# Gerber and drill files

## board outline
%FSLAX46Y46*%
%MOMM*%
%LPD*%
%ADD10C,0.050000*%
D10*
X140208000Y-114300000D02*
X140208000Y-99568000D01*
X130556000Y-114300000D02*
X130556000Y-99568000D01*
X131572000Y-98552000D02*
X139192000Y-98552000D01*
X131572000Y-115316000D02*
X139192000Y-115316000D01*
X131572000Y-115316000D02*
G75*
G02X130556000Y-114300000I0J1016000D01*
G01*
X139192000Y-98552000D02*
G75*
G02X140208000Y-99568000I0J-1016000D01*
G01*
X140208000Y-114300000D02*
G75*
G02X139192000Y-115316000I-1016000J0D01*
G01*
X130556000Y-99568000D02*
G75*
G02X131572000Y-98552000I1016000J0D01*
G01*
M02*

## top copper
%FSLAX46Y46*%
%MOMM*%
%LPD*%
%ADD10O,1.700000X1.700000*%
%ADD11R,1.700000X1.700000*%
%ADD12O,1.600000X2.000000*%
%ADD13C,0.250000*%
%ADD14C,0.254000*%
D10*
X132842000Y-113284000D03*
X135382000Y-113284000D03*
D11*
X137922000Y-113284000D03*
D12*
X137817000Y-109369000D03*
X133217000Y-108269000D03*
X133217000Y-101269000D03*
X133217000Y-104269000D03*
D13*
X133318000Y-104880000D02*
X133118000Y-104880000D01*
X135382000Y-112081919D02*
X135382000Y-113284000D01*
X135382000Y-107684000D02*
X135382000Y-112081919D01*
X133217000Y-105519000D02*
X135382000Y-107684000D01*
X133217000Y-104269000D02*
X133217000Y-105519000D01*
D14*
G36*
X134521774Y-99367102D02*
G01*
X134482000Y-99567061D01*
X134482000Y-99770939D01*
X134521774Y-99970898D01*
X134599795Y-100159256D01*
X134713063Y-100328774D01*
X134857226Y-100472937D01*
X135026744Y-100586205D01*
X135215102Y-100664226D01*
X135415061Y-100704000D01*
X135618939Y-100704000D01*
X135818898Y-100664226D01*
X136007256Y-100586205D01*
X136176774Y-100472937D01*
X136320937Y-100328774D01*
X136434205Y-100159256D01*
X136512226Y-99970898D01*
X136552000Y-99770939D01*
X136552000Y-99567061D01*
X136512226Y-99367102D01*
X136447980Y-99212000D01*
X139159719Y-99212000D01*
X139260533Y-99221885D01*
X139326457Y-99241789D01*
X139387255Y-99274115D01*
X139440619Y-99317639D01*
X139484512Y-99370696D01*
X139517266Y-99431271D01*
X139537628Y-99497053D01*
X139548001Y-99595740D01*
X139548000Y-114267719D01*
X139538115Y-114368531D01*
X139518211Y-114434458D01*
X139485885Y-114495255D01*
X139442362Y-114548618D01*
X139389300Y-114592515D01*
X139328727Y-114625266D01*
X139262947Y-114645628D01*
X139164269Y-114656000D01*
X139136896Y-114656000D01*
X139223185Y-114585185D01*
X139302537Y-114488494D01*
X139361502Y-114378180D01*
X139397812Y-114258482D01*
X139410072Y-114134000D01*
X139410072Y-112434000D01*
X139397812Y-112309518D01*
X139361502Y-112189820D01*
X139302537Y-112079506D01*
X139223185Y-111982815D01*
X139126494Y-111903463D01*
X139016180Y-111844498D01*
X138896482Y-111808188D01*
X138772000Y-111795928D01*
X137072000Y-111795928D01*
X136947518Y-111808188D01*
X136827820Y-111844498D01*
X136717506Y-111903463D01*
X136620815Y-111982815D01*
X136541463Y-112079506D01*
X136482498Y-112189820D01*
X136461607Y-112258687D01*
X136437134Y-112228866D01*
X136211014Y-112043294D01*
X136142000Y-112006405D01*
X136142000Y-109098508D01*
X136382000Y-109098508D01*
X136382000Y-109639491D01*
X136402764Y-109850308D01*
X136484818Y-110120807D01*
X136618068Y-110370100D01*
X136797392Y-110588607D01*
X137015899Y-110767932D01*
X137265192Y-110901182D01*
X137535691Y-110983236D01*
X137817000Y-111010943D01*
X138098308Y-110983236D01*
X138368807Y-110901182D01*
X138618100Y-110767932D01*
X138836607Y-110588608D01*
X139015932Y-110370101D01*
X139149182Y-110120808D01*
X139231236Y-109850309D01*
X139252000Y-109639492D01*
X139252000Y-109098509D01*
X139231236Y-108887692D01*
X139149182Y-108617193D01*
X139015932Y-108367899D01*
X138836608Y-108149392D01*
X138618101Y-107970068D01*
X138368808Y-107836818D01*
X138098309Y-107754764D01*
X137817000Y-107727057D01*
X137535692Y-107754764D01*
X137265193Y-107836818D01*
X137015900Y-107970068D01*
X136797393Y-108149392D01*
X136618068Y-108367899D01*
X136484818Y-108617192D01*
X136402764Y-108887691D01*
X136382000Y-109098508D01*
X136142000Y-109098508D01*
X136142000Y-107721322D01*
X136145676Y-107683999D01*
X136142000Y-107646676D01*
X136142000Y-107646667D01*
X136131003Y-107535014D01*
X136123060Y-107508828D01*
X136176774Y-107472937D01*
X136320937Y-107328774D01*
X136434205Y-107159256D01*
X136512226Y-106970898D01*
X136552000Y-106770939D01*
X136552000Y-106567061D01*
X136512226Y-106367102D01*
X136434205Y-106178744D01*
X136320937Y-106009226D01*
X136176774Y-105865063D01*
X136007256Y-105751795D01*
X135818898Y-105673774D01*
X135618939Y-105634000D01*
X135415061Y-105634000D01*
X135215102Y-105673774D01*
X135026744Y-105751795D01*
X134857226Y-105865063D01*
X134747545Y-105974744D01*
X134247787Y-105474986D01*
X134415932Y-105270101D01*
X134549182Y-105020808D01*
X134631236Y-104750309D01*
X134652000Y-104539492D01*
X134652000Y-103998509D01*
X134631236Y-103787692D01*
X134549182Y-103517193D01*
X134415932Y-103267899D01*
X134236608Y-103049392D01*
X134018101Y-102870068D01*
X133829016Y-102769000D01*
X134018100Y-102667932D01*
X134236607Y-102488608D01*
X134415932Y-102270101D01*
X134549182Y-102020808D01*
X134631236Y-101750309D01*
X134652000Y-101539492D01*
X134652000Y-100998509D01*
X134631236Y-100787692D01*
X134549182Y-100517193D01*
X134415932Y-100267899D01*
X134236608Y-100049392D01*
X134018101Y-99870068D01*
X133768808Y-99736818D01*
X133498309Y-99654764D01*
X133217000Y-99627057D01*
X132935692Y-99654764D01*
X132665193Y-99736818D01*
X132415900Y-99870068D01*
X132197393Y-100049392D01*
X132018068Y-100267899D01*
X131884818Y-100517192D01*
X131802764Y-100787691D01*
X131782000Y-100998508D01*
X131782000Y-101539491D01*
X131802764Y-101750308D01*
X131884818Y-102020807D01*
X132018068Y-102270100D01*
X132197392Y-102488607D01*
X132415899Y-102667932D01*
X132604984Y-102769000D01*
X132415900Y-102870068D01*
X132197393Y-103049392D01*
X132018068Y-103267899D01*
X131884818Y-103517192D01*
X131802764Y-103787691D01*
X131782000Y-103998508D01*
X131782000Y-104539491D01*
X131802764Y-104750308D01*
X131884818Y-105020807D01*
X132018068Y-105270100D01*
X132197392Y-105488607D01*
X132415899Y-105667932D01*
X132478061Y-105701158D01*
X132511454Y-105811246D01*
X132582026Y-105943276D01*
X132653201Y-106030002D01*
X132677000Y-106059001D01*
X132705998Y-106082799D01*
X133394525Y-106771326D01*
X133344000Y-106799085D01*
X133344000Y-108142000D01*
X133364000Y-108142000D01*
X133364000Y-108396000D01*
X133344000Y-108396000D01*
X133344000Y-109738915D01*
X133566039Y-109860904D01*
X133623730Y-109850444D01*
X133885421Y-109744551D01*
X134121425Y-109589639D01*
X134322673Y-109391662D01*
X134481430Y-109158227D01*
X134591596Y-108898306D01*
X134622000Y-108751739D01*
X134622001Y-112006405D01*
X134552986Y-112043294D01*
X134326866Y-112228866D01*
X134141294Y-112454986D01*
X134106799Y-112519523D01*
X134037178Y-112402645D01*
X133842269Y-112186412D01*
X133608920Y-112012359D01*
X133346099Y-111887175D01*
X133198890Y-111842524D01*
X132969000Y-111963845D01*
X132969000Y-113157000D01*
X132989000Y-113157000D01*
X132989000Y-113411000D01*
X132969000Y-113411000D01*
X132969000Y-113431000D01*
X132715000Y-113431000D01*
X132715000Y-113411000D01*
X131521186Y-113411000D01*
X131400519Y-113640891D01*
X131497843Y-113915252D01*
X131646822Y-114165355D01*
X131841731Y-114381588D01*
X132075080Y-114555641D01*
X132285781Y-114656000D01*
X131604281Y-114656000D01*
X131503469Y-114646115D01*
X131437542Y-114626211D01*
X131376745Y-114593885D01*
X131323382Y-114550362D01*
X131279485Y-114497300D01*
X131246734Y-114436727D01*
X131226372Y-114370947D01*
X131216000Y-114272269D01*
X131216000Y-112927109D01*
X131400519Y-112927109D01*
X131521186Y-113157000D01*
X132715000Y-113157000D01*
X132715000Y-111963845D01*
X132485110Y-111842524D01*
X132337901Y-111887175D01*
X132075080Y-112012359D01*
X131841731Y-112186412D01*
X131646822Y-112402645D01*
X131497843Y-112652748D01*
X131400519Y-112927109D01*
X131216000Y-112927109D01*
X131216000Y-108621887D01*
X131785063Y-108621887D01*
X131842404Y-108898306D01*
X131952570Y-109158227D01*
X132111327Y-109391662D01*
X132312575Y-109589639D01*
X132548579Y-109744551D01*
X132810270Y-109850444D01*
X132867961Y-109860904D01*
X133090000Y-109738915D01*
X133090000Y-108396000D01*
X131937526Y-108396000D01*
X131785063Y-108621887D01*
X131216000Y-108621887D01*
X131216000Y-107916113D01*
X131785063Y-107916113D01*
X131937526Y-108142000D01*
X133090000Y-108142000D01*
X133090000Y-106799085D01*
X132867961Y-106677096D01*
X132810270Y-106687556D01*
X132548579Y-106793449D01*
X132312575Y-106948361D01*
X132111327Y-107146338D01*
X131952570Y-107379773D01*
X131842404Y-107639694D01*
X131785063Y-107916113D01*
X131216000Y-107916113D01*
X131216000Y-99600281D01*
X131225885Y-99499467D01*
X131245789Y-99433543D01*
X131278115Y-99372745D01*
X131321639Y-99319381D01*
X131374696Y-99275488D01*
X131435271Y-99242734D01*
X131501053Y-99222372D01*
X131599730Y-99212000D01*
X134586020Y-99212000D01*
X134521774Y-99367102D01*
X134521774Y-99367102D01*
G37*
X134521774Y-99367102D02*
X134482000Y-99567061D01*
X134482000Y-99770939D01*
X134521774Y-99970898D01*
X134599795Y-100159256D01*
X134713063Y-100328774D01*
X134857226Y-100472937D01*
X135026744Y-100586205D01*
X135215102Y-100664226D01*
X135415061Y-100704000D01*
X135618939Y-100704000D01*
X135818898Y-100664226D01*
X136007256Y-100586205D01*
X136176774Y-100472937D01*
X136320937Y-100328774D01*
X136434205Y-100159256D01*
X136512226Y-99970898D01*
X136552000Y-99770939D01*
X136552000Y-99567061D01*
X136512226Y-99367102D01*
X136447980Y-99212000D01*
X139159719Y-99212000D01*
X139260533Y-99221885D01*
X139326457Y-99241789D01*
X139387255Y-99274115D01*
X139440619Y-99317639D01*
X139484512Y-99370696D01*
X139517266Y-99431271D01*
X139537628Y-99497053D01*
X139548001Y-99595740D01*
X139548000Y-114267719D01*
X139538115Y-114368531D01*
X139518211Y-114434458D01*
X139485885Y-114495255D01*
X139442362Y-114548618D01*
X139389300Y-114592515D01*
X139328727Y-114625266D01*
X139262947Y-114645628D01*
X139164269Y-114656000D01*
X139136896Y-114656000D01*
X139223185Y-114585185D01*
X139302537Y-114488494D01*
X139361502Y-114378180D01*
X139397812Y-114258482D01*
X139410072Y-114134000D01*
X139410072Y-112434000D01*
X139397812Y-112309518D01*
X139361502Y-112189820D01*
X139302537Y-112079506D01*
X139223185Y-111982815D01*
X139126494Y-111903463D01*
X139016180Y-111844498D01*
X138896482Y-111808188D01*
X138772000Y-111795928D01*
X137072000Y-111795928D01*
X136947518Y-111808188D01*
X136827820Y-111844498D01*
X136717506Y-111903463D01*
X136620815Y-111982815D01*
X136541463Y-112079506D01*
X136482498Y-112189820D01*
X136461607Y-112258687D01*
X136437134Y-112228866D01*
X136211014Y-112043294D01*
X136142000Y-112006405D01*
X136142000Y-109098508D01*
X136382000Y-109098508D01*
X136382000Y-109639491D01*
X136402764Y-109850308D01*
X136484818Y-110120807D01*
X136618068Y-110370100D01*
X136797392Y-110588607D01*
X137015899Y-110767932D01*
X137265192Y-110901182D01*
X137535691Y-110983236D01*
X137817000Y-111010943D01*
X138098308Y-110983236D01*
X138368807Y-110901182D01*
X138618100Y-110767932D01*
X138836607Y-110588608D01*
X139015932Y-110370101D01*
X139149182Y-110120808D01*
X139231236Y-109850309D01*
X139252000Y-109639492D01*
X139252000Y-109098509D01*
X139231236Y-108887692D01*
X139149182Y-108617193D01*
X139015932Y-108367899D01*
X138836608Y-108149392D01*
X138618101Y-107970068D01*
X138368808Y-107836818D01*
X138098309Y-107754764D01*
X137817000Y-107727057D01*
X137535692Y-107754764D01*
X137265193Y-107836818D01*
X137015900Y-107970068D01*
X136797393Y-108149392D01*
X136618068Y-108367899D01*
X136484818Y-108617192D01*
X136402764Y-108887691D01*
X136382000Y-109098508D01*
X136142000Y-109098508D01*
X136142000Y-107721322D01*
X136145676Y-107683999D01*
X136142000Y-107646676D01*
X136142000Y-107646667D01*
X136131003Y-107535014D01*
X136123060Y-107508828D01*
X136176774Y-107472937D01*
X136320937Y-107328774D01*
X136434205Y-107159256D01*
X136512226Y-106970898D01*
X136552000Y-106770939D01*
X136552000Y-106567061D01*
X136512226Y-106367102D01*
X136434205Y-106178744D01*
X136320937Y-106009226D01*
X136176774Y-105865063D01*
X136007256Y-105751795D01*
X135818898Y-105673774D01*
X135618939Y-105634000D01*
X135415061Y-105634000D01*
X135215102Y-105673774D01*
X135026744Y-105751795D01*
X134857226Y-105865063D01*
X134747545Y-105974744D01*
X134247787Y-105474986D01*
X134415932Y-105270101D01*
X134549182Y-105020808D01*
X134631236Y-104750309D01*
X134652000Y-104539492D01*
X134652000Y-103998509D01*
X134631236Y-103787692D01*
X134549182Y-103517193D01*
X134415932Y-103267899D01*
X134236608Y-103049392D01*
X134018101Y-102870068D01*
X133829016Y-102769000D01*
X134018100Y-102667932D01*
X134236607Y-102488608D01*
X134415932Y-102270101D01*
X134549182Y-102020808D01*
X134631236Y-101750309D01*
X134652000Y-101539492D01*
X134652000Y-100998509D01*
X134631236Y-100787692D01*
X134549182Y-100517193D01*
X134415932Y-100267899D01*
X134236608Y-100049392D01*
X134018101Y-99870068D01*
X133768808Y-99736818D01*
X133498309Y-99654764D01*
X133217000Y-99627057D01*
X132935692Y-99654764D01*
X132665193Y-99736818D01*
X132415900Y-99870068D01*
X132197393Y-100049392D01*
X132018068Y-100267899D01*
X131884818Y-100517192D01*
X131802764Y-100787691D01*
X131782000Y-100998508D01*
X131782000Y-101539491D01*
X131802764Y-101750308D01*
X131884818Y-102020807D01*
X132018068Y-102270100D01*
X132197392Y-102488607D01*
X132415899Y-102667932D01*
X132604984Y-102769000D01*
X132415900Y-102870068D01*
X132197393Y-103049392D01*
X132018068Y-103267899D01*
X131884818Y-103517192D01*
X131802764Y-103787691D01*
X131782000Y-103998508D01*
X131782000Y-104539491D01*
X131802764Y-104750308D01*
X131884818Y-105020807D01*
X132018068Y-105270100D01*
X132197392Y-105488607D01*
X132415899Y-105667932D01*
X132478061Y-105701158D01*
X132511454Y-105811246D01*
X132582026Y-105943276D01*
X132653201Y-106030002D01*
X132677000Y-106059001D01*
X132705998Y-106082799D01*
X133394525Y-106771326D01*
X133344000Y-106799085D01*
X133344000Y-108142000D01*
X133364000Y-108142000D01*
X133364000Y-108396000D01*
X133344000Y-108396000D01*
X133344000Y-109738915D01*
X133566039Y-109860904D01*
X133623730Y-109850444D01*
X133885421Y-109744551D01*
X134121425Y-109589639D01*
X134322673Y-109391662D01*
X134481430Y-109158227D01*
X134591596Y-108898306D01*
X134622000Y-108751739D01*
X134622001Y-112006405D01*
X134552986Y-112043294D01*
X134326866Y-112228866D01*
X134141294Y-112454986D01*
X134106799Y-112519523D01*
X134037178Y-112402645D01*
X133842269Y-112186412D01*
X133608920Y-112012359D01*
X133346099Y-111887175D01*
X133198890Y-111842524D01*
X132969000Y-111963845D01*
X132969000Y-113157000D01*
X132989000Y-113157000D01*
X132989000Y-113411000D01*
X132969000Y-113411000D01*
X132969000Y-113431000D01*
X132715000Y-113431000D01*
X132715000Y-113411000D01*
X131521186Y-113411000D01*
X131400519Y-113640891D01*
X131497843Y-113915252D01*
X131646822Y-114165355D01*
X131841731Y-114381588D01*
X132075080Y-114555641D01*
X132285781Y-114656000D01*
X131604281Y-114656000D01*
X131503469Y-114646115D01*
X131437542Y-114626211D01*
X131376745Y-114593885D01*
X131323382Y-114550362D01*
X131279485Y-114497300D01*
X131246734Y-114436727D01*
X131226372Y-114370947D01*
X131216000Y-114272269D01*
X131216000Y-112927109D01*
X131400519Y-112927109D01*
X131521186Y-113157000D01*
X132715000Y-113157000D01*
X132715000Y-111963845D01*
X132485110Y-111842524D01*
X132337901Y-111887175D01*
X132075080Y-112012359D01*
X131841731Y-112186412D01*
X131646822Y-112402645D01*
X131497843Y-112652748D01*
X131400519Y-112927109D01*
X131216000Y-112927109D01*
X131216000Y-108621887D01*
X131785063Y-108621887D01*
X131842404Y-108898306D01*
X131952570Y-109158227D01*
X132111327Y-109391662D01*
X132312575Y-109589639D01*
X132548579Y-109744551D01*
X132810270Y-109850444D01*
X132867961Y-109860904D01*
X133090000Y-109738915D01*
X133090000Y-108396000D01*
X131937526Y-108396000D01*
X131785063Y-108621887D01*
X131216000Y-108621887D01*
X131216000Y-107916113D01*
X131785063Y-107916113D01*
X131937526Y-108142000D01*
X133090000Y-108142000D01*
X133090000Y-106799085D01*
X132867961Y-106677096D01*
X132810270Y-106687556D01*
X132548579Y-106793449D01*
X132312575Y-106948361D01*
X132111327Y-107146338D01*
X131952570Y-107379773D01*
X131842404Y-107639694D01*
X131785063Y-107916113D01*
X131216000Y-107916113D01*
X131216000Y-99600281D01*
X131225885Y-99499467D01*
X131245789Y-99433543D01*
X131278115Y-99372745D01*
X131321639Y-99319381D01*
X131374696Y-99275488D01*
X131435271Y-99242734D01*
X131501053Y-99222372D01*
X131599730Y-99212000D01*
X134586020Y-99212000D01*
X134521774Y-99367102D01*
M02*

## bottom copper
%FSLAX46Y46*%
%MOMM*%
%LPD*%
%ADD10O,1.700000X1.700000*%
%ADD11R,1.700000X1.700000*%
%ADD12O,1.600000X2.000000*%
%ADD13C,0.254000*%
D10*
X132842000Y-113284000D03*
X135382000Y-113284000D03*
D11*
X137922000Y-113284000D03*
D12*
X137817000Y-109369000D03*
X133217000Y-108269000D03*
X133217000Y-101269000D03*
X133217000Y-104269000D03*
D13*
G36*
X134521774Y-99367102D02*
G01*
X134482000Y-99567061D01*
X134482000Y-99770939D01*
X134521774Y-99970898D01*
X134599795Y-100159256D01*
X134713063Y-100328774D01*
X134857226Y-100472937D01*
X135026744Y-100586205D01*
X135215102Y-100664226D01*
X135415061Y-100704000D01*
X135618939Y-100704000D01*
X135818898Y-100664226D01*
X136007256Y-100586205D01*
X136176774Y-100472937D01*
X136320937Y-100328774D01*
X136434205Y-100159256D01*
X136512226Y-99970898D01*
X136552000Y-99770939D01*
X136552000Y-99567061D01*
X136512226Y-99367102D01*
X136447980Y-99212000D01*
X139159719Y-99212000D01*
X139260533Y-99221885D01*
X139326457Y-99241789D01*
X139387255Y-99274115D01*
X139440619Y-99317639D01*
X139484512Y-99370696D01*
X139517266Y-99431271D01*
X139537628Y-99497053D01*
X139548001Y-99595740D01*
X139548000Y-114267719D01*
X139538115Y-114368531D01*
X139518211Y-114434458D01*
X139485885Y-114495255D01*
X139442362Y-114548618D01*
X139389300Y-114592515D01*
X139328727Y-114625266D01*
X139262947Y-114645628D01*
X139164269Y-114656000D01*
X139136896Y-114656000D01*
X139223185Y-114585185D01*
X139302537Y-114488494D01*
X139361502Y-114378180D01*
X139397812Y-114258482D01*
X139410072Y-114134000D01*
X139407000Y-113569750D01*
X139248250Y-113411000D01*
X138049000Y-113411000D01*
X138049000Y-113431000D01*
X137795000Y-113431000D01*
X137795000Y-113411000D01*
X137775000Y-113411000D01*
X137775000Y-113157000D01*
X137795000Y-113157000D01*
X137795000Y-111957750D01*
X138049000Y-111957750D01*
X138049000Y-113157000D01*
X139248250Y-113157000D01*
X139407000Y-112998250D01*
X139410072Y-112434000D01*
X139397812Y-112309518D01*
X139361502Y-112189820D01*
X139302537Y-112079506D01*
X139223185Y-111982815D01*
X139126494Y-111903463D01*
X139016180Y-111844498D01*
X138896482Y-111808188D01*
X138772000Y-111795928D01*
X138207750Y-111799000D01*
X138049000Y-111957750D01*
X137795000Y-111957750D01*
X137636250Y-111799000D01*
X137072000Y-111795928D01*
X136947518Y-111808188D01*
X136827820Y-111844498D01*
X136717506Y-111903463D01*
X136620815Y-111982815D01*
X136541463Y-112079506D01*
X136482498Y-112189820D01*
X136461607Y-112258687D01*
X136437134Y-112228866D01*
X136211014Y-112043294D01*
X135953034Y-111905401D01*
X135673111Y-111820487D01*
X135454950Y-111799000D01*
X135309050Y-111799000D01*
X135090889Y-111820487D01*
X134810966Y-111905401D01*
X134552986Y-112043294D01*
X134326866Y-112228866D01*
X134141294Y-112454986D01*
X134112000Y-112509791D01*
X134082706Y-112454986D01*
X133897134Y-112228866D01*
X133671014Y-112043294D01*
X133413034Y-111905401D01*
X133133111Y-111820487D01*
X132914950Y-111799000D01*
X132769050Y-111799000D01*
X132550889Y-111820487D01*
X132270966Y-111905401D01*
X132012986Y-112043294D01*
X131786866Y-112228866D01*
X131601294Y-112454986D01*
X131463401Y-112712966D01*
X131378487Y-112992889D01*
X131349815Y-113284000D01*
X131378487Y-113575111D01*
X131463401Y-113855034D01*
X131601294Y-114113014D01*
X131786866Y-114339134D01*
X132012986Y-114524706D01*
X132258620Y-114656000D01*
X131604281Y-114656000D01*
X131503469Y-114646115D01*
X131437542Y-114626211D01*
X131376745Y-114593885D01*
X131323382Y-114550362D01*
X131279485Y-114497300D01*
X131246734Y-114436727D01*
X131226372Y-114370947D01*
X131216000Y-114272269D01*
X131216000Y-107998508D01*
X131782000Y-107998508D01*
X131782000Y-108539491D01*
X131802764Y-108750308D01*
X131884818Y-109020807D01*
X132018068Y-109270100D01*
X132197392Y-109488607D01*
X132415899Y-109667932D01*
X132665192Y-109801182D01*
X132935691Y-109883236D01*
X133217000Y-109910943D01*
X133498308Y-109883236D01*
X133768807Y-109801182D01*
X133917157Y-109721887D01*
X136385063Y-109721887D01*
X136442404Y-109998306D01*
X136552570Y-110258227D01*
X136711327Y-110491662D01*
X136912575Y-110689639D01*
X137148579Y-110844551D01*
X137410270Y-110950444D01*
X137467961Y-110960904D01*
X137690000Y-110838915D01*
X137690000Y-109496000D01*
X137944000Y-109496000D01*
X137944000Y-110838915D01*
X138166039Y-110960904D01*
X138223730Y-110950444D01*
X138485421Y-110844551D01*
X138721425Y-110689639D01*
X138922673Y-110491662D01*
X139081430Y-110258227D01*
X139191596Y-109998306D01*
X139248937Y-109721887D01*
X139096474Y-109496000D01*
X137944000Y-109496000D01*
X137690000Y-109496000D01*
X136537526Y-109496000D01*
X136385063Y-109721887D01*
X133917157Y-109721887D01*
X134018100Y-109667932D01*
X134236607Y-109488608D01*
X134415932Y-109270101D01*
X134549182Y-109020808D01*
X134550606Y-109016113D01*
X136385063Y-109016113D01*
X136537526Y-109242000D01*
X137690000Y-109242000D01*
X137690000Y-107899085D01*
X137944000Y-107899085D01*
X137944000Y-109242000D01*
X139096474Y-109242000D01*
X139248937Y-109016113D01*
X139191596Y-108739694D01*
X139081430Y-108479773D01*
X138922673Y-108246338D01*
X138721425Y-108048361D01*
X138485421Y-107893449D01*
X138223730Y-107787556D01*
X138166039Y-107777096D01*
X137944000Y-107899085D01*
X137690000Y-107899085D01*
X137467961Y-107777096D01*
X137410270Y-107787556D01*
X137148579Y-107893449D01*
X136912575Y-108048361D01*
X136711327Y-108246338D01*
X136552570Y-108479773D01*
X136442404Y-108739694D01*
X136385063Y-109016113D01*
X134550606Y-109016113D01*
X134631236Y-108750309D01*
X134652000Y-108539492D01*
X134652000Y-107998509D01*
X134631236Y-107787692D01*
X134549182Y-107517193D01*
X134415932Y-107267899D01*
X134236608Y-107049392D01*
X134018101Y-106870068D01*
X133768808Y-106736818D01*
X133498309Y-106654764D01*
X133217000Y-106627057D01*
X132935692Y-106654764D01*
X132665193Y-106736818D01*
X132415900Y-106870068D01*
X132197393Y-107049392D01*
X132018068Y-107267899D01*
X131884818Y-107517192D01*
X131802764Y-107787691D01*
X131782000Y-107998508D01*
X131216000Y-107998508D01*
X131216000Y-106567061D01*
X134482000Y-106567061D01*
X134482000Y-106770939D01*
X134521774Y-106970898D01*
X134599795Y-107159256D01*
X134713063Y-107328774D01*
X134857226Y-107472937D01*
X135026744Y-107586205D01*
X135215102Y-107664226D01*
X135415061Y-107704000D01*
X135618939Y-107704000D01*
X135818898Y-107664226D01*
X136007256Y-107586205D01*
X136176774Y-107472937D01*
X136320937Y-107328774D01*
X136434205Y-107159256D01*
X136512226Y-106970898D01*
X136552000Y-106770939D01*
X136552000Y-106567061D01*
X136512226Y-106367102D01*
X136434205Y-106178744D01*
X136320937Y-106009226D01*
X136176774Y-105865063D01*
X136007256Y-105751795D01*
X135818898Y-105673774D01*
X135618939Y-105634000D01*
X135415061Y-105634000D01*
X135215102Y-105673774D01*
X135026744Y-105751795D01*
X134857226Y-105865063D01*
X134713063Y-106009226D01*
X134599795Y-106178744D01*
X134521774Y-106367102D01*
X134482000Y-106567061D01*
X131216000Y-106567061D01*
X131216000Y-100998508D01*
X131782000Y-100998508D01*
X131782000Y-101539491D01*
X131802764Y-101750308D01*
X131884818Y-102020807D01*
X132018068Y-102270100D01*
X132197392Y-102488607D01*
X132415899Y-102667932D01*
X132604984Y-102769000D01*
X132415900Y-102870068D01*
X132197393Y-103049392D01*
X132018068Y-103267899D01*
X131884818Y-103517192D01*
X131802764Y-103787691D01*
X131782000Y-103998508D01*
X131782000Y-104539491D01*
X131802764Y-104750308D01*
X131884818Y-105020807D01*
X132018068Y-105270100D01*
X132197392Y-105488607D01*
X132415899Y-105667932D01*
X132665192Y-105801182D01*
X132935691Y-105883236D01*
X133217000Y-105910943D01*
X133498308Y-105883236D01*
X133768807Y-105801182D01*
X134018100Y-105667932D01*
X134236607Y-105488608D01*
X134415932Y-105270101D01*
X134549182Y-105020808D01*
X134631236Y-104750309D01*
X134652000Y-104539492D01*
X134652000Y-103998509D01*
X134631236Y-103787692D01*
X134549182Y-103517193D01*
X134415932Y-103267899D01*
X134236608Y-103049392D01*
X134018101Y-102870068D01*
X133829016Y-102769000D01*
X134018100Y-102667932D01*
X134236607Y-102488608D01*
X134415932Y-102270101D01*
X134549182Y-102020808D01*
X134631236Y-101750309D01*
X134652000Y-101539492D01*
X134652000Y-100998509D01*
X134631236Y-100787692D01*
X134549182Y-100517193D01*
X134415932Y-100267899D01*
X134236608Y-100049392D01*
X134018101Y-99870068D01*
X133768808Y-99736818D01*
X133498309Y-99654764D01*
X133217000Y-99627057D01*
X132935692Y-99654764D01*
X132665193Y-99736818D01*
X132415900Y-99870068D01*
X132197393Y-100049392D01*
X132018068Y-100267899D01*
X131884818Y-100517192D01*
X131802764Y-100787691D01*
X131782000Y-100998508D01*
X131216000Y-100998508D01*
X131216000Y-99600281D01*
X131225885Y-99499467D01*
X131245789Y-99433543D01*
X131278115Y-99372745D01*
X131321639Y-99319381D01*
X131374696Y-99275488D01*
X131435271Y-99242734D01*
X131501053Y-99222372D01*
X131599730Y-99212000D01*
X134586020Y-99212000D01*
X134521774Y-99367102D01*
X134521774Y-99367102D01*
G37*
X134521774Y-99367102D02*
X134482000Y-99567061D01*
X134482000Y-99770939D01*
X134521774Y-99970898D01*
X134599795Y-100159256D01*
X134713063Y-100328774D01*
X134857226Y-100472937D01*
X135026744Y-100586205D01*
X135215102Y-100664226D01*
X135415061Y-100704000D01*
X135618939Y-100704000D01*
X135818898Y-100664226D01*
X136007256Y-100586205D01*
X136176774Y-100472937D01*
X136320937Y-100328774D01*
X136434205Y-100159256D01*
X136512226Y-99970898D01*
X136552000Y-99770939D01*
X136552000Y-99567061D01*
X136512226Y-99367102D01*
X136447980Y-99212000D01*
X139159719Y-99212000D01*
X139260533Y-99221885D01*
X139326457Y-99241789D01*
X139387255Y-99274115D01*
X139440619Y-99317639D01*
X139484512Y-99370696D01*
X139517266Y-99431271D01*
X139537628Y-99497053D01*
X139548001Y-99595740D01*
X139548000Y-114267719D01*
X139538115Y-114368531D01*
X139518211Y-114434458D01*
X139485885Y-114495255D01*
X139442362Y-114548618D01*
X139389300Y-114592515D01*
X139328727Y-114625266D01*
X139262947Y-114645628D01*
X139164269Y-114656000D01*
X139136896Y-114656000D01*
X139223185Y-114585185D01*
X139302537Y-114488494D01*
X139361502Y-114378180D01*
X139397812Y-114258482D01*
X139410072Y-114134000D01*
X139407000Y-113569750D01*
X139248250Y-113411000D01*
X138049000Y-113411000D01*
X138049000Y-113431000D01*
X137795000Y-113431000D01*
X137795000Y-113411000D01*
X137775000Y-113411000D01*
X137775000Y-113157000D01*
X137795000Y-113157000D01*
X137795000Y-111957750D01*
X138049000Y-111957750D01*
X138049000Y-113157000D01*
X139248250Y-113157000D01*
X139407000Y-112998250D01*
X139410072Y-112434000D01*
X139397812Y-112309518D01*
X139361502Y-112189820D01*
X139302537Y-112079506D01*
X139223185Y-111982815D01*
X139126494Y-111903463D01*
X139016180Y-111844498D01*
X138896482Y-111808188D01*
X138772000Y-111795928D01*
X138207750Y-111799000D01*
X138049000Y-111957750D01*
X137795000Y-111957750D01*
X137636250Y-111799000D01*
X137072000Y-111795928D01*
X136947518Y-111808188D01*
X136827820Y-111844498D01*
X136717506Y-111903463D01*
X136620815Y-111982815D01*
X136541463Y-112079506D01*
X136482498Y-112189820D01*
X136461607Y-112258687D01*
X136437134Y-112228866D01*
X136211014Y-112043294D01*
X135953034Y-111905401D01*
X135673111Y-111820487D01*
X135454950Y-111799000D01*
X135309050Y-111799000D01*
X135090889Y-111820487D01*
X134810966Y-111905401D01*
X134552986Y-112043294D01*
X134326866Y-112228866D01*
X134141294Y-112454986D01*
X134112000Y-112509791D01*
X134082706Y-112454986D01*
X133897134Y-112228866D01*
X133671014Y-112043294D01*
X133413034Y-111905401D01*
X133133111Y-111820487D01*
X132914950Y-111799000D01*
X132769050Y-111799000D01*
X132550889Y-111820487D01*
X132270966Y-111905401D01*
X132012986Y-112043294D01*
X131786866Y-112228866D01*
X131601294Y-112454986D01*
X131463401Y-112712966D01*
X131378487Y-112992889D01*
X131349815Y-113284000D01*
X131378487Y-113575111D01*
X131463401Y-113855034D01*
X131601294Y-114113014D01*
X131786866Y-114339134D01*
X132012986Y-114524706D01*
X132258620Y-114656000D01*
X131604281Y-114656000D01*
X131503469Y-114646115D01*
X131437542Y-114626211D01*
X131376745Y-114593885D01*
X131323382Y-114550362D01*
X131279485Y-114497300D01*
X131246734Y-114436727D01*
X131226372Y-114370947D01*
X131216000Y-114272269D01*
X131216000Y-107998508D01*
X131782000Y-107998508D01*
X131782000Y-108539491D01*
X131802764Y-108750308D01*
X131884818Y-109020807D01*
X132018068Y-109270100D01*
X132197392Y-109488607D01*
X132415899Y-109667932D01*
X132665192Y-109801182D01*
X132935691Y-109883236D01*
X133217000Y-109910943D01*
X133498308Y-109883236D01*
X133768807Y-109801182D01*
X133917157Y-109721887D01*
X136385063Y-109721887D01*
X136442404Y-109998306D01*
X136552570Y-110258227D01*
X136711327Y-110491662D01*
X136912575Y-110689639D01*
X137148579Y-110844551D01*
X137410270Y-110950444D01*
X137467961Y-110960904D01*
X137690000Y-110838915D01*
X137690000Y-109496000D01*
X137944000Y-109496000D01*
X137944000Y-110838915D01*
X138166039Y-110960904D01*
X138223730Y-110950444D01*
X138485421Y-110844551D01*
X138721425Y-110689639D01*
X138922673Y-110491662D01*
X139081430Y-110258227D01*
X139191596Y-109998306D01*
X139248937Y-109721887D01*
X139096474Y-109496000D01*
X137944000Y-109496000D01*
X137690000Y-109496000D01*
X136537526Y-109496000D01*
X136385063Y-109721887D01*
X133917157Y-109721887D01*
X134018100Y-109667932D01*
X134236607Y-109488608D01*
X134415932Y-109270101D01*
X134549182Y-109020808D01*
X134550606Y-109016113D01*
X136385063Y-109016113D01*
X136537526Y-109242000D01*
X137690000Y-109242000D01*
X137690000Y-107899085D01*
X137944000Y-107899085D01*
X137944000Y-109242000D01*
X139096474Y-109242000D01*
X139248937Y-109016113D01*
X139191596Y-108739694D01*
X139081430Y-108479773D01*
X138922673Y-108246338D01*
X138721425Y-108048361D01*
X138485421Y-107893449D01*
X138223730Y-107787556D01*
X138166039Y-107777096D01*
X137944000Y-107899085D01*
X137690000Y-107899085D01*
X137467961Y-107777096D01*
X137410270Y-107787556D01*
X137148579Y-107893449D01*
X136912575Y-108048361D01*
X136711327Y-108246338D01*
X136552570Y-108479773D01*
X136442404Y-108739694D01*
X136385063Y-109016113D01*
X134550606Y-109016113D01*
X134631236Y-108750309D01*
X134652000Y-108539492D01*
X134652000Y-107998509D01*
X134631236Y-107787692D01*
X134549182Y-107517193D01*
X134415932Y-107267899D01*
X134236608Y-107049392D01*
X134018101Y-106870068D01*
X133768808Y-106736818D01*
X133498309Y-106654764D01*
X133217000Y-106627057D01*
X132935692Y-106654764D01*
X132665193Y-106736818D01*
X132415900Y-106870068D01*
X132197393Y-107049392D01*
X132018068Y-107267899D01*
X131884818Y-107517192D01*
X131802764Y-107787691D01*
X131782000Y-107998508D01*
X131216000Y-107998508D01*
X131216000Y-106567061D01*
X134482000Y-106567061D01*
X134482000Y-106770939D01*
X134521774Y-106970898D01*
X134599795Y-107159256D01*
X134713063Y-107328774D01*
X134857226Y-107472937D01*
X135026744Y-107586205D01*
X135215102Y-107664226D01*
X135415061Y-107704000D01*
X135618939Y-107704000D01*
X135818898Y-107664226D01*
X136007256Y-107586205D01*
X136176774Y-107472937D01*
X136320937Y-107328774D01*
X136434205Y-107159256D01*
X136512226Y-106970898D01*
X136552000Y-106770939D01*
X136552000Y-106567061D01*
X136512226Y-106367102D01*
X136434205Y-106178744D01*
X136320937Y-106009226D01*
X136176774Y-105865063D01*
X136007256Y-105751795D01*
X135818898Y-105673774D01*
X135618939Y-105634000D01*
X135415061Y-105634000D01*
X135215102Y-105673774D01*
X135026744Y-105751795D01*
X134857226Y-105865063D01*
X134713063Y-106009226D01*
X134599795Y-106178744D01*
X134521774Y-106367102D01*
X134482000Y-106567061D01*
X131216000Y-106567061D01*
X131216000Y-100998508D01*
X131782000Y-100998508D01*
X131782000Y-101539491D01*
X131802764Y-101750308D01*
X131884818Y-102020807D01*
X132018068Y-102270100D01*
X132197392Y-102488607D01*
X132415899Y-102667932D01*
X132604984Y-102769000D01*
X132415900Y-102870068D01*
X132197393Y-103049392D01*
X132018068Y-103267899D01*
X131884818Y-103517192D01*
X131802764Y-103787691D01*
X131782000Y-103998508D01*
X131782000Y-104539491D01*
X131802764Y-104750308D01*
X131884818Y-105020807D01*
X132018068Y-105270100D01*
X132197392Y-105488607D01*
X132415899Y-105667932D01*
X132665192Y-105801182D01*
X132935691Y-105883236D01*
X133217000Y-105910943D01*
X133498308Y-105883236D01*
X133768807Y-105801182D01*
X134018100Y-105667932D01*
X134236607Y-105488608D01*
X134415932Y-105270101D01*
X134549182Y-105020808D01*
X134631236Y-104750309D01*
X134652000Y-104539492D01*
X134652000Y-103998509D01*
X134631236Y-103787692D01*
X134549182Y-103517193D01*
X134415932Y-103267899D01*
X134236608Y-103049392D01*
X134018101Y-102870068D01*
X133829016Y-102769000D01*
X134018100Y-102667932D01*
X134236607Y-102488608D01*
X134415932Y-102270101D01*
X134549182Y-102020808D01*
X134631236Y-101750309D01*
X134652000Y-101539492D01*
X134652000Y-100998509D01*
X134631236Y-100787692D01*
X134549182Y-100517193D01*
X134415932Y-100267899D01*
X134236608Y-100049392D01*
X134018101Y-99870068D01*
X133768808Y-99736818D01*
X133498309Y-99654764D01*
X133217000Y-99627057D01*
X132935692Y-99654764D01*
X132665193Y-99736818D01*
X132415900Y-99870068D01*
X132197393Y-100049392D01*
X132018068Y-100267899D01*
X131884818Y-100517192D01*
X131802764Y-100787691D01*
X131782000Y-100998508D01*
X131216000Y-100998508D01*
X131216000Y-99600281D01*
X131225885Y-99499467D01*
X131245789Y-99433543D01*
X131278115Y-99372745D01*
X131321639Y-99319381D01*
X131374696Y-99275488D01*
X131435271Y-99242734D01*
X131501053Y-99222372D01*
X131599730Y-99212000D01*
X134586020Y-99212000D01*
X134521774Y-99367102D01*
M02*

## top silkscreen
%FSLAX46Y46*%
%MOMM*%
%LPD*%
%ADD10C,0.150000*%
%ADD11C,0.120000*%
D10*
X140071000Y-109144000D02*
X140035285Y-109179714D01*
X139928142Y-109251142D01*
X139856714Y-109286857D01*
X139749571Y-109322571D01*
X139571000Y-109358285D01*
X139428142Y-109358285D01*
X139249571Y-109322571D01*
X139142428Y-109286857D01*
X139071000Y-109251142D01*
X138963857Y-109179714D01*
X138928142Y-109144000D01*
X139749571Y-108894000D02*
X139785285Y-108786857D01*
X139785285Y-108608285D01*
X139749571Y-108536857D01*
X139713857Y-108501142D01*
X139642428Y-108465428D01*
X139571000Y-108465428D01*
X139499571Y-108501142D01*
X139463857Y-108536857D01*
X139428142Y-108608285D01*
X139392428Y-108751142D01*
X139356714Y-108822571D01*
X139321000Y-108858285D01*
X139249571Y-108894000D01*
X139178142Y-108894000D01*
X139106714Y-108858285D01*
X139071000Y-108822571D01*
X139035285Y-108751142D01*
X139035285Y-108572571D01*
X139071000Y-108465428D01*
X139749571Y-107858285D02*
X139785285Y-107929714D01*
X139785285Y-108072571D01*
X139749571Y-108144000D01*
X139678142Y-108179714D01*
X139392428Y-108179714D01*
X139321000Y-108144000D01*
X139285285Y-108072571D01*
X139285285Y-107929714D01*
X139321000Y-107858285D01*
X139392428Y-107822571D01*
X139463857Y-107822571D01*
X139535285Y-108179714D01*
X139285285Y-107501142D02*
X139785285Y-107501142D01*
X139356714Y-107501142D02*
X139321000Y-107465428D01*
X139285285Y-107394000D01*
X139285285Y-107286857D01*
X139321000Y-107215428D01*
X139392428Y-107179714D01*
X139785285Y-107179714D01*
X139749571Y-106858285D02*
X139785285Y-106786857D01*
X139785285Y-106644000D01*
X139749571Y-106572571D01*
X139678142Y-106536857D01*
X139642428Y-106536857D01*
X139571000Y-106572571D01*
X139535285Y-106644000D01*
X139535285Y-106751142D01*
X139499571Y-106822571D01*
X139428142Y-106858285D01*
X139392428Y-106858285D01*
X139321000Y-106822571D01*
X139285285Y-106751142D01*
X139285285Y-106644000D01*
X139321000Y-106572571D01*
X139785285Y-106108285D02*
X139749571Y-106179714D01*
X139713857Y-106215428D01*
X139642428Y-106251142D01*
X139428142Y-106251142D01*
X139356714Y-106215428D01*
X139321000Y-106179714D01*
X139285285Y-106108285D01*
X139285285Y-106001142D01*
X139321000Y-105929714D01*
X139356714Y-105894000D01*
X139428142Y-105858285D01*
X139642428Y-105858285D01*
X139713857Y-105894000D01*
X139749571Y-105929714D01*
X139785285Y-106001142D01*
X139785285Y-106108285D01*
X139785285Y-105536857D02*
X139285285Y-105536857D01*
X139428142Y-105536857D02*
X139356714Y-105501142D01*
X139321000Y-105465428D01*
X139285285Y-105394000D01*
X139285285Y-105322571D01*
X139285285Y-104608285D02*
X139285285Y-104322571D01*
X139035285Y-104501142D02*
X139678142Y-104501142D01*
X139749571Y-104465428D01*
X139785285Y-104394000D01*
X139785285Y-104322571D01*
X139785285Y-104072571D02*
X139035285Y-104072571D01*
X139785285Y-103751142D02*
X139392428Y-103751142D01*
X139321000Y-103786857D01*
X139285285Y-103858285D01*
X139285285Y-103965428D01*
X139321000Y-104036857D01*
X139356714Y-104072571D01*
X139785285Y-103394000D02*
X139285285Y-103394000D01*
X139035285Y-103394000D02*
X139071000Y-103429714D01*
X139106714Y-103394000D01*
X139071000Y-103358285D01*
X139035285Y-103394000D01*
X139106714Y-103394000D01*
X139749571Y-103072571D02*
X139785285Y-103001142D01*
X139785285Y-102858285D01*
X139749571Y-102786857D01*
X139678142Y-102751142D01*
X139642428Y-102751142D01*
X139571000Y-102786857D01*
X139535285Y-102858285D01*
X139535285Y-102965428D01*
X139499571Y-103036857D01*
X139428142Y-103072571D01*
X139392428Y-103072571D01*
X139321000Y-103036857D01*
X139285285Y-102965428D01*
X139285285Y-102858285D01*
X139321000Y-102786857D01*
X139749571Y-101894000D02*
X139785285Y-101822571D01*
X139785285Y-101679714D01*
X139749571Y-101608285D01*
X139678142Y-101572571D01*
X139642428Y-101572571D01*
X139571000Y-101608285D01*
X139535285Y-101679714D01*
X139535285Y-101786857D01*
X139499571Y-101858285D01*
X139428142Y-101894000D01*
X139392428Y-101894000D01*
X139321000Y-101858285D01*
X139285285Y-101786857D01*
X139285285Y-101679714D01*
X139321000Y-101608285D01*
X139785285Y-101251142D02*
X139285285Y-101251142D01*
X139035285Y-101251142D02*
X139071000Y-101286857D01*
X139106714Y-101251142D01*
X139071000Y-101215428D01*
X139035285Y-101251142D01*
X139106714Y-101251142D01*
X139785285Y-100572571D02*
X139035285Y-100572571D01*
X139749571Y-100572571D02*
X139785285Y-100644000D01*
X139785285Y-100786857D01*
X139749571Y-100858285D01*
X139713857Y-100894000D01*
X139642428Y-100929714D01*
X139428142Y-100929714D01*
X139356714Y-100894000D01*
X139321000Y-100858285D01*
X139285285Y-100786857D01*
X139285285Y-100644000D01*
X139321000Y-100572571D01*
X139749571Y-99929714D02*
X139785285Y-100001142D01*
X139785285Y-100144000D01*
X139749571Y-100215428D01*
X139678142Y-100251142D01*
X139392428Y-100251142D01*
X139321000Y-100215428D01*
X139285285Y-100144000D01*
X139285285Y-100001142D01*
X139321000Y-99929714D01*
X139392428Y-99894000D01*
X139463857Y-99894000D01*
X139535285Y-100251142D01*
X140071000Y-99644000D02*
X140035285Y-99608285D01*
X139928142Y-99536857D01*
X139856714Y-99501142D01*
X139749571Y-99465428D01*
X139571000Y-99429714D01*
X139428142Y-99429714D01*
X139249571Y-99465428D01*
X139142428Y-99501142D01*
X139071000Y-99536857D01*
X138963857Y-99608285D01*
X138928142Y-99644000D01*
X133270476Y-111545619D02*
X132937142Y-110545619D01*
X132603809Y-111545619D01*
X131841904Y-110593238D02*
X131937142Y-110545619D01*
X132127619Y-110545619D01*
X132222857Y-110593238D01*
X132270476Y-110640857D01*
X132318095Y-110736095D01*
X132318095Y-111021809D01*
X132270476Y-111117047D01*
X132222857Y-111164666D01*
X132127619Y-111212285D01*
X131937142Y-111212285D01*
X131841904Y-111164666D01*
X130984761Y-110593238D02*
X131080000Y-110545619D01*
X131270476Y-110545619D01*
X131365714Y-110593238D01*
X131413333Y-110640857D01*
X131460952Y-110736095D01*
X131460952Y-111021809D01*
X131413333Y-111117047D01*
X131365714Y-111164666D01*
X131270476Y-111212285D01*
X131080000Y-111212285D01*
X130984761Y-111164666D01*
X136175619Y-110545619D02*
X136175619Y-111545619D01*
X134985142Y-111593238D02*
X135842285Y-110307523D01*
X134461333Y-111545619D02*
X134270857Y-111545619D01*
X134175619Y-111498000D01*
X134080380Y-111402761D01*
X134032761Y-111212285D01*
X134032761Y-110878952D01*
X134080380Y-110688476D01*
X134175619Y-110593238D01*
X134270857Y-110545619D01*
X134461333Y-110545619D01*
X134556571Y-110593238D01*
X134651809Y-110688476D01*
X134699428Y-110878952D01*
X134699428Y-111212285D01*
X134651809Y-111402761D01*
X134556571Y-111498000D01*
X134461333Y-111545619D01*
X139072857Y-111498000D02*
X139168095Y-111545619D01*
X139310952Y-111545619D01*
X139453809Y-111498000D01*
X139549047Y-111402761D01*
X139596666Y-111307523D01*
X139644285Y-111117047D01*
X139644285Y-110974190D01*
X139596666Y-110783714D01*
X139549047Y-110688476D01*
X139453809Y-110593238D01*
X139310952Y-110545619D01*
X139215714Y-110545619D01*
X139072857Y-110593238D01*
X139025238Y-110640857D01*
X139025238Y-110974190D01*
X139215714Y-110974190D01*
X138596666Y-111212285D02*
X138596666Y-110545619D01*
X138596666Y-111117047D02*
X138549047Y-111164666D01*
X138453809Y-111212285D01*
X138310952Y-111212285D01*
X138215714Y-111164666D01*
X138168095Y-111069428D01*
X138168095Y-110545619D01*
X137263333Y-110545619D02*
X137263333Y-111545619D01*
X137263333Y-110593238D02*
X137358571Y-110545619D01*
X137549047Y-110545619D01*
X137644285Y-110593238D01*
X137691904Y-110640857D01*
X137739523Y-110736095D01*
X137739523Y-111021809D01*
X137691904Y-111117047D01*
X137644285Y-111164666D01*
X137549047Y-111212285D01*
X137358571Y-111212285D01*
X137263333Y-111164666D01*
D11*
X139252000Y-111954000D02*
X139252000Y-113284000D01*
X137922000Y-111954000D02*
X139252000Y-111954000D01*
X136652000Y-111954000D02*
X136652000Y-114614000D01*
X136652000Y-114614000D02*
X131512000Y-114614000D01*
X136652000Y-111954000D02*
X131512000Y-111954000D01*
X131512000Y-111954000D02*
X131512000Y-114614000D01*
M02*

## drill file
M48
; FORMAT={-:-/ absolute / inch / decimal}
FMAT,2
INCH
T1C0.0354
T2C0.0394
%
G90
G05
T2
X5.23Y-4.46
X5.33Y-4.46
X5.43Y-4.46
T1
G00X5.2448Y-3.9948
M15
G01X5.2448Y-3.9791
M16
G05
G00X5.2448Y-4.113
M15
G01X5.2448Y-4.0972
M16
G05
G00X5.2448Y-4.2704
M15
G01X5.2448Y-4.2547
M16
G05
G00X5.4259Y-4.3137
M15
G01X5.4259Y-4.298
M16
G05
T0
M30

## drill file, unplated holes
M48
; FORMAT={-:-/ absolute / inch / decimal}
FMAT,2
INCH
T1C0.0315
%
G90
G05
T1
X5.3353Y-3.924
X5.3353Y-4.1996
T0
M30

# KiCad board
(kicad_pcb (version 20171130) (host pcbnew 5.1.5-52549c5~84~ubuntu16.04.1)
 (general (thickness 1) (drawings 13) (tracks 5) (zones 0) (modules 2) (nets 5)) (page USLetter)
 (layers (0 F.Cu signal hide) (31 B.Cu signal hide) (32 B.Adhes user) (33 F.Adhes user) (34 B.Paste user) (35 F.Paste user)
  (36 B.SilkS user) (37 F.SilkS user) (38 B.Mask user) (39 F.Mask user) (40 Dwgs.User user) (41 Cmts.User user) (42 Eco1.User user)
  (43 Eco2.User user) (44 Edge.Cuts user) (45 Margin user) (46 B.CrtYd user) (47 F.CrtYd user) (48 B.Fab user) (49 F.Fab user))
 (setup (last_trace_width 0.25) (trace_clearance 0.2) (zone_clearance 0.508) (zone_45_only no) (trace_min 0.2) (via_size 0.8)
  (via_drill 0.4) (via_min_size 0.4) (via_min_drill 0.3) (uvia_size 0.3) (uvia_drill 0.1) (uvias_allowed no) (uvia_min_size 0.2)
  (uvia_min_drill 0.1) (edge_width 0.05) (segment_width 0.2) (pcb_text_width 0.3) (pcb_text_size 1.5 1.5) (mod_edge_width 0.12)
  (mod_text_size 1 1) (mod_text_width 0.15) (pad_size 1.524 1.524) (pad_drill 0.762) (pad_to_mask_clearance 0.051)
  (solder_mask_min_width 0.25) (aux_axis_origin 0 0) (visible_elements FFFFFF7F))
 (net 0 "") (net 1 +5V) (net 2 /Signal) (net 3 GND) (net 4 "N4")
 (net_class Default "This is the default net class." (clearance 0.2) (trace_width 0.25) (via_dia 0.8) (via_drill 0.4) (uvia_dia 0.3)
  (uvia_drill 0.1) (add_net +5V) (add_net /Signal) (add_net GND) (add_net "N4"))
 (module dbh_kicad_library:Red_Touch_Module (layer F.Cu) (at 137.922 113.284 270)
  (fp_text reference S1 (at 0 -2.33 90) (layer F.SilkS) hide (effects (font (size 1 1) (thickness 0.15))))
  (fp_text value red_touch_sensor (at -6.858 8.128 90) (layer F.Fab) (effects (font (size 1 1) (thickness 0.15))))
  (fp_line (start -1.33 -1.33) (end 0 -1.33) (layer F.SilkS) (width 0.12))
  (fp_line (start -1.33 0) (end -1.33 -1.33) (layer F.SilkS) (width 0.12))
  (fp_line (start -1.33 1.27) (end 1.33 1.27) (layer F.SilkS) (width 0.12))
  (fp_line (start 1.33 1.27) (end 1.33 6.41) (layer F.SilkS) (width 0.12))
  (fp_line (start -1.33 1.27) (end -1.33 6.41) (layer F.SilkS) (width 0.12))
  (fp_line (start -1.33 6.41) (end 1.33 6.41) (layer F.SilkS) (width 0.12))
  (pad 3 thru_hole oval (at 0 5.08 270) (size 1.7 1.7) (drill 1) (layers *.Cu *.Mask) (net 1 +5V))
  (pad 2 thru_hole oval (at 0 2.54 270) (size 1.7 1.7) (drill 1) (layers *.Cu *.Mask) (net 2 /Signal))
  (pad 1 thru_hole rect (at 0 0 270) (size 1.7 1.7) (drill 1) (layers *.Cu *.Mask) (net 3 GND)))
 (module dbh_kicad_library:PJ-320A (layer B.Cu) (at 133.477 101.219 270)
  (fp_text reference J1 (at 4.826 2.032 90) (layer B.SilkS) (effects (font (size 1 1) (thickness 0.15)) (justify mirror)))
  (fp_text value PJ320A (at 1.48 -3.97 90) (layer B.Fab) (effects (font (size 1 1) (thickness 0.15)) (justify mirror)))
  (pad 5 thru_hole oval (at 8.15 -4.34 180) (size 1.6 2) (drill oval 0.9 1.3) (layers *.Cu *.Mask) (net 3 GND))
  (pad 4 thru_hole oval (at 7.05 0.26 180) (size 1.6 2) (drill oval 0.9 1.3) (layers *.Cu *.Mask) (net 1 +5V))
  (pad 2 thru_hole oval (at 0.05 0.26 180) (size 1.6 2) (drill oval 0.9 1.3) (layers *.Cu *.Mask) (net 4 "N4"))
  (pad "" np_thru_hole circle (at 5.45 -2.04 180) (size 0.8 0.8) (drill 0.8) (layers *.Cu *.Mask))
  (pad "" np_thru_hole circle (at -1.55 -2.04 180) (size 0.8 0.8) (drill 0.8) (layers *.Cu *.Mask))
  (pad 3 thru_hole oval (at 3.05 0.26 180) (size 1.6 2) (drill oval 0.9 1.3) (layers *.Cu *.Mask) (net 2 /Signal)))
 (gr_line (start 140.208 114.3) (end 140.208 99.568) (layer Edge.Cuts) (width 0.05))
 (gr_line (start 130.556 114.3) (end 130.556 99.568) (layer Edge.Cuts) (width 0.05))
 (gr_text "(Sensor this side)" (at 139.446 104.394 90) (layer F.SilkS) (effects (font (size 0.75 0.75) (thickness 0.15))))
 (gr_line (start 131.572 98.552) (end 139.192 98.552) (layer Edge.Cuts) (width 0.05))
 (gr_line (start 131.572 115.316) (end 139.192 115.316) (layer Edge.Cuts) (width 0.05))
 (gr_arc (start 131.572 114.3) (end 130.556 114.3) (angle -90) (layer Edge.Cuts) (width 0.05))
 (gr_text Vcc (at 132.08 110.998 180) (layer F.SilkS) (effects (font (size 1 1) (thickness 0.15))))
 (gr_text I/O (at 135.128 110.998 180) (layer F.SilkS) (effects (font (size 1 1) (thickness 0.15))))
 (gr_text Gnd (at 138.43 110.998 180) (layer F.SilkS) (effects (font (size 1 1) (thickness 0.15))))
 (gr_arc (start 139.192 99.568) (end 140.208 99.568) (angle -90) (layer Edge.Cuts) (width 0.05))
 (gr_arc (start 139.192 114.3) (end 139.192 115.316) (angle -90) (layer Edge.Cuts) (width 0.05))
 (gr_arc (start 131.572 99.568) (end 131.572 98.552) (angle -90) (layer Edge.Cuts) (width 0.05))
 (segment (start 133.318 104.88) (end 133.118 104.88) (width 0.25) (layer F.Cu) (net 2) (status 30))
 (segment (start 135.382 112.081919) (end 135.382 113.284) (width 0.25) (layer F.Cu) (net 2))
 (segment (start 135.382 107.684) (end 135.382 112.081919) (width 0.25) (layer F.Cu) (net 2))
 (segment (start 133.217 105.519) (end 135.382 107.684) (width 0.25) (layer F.Cu) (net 2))
 (segment (start 133.217 104.269) (end 133.217 105.519) (width 0.25) (layer F.Cu) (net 2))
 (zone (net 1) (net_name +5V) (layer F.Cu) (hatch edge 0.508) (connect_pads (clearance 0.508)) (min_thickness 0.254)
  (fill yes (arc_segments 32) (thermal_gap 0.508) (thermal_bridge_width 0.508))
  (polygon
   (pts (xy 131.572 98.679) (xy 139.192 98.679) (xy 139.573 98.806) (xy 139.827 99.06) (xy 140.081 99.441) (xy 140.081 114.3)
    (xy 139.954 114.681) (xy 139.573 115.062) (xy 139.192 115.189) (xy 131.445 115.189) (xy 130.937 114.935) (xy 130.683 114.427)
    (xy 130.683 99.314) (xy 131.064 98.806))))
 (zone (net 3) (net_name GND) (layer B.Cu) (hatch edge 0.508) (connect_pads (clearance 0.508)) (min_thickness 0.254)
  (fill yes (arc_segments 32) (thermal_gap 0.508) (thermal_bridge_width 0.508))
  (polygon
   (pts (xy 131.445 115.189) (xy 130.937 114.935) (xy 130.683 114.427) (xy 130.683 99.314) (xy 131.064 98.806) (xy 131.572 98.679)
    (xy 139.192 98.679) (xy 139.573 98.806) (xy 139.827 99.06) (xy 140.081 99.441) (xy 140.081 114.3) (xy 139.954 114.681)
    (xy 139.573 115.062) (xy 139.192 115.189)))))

